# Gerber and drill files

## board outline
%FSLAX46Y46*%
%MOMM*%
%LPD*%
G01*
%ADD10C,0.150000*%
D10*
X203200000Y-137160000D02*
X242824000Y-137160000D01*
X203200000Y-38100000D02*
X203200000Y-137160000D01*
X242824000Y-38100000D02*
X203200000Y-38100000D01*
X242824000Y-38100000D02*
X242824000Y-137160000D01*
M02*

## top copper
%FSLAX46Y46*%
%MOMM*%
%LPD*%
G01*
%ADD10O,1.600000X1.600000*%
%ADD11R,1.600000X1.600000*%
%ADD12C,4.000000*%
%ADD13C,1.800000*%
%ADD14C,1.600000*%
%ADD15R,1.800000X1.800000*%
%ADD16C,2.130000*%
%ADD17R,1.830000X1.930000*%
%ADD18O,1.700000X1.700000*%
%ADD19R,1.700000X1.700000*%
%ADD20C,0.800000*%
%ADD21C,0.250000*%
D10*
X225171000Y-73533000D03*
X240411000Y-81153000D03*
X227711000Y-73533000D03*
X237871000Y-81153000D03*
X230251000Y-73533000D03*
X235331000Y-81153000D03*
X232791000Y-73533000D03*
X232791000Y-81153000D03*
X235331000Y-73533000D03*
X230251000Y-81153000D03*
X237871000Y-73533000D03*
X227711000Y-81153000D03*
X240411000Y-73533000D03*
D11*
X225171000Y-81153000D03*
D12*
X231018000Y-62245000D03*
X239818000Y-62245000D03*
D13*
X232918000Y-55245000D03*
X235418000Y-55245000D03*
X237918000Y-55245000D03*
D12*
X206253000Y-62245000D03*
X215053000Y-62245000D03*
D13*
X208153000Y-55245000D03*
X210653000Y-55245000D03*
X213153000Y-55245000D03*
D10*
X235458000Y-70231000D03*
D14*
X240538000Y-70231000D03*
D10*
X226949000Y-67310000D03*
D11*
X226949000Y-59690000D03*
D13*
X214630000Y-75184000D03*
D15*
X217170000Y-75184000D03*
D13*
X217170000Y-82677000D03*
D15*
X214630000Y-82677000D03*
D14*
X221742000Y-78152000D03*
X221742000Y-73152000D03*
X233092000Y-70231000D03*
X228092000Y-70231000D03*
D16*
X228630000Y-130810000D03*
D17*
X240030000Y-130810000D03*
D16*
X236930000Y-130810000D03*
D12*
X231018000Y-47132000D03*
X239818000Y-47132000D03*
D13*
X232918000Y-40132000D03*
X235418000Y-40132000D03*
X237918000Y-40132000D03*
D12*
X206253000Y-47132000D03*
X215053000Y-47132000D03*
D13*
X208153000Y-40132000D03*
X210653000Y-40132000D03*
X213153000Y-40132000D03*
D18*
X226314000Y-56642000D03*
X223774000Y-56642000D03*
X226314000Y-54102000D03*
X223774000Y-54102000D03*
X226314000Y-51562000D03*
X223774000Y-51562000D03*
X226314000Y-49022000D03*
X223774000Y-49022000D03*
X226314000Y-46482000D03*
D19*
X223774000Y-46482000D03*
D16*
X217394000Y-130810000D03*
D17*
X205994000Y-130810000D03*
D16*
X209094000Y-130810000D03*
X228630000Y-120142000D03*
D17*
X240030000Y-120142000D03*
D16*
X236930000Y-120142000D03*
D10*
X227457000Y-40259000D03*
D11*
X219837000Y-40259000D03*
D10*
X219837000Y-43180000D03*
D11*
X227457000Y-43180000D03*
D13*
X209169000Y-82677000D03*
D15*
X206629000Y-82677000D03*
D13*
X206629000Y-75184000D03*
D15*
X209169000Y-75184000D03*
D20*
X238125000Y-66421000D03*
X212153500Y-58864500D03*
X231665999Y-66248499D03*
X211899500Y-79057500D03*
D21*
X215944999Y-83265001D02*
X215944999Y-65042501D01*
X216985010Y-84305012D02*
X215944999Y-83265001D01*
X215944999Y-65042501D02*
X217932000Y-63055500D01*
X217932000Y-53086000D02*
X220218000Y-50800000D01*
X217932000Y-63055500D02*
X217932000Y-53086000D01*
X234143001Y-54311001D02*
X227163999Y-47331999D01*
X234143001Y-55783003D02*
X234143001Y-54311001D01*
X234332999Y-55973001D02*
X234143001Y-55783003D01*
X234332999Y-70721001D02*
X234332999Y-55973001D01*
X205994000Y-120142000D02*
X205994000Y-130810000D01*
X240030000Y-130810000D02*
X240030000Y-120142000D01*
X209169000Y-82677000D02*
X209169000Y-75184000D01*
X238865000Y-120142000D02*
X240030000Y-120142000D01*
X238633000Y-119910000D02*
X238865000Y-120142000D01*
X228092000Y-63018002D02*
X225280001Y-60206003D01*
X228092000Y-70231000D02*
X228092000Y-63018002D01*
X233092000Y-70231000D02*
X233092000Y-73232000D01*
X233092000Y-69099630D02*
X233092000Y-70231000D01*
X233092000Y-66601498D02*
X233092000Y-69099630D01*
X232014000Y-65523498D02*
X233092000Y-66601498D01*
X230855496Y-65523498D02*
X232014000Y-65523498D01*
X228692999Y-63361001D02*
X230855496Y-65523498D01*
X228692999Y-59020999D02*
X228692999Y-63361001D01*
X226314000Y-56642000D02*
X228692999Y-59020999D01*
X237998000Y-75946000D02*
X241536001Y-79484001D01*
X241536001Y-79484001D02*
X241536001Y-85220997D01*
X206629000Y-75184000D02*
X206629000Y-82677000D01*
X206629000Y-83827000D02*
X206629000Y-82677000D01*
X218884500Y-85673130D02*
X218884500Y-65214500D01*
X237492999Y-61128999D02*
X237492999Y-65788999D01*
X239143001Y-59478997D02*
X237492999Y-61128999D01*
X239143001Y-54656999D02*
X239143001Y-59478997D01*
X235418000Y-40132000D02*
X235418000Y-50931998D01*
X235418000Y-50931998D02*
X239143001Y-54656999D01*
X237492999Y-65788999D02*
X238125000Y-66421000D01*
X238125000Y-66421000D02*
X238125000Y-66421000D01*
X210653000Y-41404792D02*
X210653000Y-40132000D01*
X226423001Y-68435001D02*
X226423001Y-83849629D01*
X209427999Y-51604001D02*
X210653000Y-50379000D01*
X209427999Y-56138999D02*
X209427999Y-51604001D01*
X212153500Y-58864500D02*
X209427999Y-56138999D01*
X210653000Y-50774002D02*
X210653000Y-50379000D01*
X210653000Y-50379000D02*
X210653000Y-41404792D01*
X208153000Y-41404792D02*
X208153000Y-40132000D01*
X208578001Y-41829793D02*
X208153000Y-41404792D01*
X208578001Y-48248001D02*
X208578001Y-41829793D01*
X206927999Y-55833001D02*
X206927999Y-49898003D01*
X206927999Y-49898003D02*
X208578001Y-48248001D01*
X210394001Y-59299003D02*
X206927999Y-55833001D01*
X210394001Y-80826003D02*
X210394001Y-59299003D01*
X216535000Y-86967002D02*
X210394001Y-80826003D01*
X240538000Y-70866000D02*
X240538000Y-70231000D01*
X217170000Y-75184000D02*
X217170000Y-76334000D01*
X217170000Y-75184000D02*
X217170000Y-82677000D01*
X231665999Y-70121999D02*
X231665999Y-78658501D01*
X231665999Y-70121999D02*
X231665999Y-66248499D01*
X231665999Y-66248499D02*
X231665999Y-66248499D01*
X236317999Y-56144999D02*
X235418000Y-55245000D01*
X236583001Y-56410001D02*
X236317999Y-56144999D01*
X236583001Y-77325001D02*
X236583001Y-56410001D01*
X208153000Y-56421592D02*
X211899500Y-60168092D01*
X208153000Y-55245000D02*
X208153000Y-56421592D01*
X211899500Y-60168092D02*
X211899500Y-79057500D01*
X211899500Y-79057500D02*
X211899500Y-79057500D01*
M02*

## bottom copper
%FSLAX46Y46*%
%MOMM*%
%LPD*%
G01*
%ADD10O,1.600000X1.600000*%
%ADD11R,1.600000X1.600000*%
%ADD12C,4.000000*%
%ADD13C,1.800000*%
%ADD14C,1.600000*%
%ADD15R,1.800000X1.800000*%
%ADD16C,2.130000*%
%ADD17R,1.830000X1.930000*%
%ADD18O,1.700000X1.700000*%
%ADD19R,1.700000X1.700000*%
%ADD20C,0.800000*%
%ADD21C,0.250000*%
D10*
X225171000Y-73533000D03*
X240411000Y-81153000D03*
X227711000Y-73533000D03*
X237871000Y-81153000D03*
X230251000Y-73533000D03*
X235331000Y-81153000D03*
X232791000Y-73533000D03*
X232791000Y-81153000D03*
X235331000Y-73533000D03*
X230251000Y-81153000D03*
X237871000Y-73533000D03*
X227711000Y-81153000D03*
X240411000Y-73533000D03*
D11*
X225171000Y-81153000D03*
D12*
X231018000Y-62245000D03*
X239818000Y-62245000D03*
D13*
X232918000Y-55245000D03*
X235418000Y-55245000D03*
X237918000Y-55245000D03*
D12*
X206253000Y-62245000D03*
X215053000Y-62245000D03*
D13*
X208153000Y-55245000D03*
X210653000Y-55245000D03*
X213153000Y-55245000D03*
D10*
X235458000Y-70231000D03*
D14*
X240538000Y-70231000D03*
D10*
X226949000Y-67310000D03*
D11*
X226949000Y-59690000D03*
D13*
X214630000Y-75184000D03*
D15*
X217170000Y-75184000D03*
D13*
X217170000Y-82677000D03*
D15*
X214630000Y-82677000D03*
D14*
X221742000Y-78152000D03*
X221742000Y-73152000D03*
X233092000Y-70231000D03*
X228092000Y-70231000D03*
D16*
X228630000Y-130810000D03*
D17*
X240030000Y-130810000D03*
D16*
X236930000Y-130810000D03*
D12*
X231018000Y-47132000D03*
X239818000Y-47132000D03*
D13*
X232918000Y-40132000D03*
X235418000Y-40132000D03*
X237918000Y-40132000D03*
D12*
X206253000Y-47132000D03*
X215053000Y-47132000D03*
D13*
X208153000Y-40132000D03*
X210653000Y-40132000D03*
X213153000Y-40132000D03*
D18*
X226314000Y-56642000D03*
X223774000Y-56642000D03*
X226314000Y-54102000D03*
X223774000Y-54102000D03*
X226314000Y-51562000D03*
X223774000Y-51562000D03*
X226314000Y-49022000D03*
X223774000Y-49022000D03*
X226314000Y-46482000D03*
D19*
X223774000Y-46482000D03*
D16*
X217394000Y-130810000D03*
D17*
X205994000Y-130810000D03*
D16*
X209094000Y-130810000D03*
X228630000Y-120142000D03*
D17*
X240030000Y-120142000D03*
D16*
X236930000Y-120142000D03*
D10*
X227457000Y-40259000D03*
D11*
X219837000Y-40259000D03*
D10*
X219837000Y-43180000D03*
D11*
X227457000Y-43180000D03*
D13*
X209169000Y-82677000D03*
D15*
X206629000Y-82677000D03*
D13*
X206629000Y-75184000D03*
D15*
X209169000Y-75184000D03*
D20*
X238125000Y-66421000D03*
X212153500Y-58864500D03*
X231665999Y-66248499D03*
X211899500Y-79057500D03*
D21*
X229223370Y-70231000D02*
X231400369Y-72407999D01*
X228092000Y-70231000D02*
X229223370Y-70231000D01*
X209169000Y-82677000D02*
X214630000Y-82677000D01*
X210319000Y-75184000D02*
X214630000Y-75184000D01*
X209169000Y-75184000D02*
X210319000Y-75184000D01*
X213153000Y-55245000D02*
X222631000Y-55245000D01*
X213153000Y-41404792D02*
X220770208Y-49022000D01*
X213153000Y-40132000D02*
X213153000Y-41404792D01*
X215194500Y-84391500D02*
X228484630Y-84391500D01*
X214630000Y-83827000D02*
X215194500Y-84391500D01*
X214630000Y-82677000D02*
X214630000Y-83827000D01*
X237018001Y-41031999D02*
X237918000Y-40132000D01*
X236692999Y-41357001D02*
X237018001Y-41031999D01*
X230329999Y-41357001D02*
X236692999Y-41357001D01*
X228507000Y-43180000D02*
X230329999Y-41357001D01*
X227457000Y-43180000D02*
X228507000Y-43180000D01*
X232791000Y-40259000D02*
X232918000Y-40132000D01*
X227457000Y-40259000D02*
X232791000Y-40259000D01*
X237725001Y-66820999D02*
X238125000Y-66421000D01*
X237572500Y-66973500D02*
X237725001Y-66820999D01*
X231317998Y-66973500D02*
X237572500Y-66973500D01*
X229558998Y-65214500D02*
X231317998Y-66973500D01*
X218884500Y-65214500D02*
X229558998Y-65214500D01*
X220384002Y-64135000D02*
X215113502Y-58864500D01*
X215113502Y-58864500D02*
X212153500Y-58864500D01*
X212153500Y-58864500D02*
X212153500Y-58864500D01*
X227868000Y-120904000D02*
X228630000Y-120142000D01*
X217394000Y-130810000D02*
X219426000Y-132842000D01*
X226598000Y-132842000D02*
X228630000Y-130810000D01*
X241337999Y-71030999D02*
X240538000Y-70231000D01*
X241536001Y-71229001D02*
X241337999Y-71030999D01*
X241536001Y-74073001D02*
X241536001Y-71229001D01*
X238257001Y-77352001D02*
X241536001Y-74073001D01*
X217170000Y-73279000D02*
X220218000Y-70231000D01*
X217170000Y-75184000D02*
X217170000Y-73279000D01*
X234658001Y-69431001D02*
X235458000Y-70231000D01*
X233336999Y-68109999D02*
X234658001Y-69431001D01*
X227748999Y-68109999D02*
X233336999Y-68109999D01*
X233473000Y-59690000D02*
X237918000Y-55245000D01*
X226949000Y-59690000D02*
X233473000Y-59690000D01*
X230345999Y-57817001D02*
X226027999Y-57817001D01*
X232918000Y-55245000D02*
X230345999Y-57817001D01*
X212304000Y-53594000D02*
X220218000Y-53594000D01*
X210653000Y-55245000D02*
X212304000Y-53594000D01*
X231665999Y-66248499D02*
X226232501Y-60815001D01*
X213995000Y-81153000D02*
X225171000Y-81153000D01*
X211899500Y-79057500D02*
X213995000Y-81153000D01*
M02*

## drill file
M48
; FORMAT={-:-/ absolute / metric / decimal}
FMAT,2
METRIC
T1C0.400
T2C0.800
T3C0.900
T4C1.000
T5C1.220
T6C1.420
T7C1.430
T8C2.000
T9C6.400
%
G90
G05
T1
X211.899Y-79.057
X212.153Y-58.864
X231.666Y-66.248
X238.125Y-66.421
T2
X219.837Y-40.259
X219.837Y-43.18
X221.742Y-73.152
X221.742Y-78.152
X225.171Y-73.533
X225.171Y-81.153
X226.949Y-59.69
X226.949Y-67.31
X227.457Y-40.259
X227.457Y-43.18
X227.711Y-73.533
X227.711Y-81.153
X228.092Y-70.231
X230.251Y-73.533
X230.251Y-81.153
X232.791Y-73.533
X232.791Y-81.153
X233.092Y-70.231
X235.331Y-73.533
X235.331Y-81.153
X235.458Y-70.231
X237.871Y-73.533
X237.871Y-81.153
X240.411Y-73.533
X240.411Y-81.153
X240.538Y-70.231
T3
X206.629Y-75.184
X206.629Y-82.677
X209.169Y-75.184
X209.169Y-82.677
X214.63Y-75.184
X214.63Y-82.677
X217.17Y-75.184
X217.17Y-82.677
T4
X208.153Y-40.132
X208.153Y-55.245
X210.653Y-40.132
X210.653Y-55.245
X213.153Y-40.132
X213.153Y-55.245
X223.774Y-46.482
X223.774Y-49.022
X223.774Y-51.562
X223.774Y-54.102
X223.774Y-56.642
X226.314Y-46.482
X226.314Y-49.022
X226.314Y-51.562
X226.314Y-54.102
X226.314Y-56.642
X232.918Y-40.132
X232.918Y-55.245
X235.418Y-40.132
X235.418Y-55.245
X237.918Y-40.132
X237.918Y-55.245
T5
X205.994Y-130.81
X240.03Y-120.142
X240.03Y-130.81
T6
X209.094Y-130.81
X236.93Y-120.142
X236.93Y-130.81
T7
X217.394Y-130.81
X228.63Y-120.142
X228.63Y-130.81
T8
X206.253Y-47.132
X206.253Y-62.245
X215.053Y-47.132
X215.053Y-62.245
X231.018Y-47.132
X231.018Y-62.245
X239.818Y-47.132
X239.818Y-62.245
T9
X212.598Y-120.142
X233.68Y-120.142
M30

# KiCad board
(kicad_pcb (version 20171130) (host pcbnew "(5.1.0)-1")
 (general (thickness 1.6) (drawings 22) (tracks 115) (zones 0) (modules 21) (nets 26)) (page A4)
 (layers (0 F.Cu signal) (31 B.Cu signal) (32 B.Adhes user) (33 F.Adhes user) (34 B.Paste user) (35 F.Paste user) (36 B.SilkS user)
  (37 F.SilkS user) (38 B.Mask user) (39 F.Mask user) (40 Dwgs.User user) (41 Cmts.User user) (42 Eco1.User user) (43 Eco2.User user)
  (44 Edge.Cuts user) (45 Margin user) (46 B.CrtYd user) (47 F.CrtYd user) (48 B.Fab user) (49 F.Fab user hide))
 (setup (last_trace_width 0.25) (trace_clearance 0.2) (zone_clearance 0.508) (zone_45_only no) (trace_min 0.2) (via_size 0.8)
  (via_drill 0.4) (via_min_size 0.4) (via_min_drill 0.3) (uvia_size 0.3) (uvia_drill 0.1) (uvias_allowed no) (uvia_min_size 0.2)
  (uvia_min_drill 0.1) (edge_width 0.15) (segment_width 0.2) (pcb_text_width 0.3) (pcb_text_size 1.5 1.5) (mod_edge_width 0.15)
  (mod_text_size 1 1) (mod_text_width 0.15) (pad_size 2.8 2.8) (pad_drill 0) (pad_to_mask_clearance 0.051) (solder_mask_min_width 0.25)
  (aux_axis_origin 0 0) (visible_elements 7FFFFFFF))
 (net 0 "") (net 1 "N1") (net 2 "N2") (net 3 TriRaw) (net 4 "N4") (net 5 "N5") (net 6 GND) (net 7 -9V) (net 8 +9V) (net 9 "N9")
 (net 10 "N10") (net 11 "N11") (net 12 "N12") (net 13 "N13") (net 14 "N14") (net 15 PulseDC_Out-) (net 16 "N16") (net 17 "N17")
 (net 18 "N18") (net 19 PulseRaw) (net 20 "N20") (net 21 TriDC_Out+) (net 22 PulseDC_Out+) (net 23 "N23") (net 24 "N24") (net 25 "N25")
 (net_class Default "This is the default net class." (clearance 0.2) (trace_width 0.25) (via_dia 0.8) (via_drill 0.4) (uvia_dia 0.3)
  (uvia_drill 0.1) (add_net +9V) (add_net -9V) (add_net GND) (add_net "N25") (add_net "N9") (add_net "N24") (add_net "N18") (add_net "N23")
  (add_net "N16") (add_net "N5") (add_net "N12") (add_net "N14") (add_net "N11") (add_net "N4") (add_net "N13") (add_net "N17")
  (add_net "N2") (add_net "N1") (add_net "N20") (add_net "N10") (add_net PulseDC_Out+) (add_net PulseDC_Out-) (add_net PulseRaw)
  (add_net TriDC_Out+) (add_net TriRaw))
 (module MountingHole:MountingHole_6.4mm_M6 (layer F.Cu) (at 233.68 120.142)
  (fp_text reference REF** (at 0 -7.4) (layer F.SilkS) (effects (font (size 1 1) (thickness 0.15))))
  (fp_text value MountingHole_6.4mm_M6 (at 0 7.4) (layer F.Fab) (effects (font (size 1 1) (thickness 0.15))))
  (pad 1 np_thru_hole circle (at 0 0) (size 6.4 6.4) (drill 6.4) (layers *.Cu *.Mask)))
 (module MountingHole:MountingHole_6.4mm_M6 (layer F.Cu) (at 212.598 120.142)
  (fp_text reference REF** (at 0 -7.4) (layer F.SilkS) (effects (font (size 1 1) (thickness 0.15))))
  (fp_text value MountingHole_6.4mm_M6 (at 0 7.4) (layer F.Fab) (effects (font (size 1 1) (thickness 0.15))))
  (pad 1 np_thru_hole circle (at 0 0) (size 6.4 6.4) (drill 6.4) (layers *.Cu *.Mask)))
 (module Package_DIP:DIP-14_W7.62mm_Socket (layer F.Cu) (at 225.171 81.153 90)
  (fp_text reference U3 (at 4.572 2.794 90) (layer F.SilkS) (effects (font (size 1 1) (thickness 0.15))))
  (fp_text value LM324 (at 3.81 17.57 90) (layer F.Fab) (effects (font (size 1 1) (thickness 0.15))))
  (pad 14 thru_hole oval (at 7.62 0 90) (size 1.6 1.6) (drill 0.8) (layers *.Cu *.Mask) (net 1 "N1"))
  (pad 7 thru_hole oval (at 0 15.24 90) (size 1.6 1.6) (drill 0.8) (layers *.Cu *.Mask) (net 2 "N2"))
  (pad 13 thru_hole oval (at 7.62 2.54 90) (size 1.6 1.6) (drill 0.8) (layers *.Cu *.Mask) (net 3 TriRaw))
  (pad 6 thru_hole oval (at 0 12.7 90) (size 1.6 1.6) (drill 0.8) (layers *.Cu *.Mask) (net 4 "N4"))
  (pad 12 thru_hole oval (at 7.62 5.08 90) (size 1.6 1.6) (drill 0.8) (layers *.Cu *.Mask) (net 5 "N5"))
  (pad 5 thru_hole oval (at 0 10.16 90) (size 1.6 1.6) (drill 0.8) (layers *.Cu *.Mask) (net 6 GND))
  (pad 11 thru_hole oval (at 7.62 7.62 90) (size 1.6 1.6) (drill 0.8) (layers *.Cu *.Mask) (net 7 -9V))
  (pad 4 thru_hole oval (at 0 7.62 90) (size 1.6 1.6) (drill 0.8) (layers *.Cu *.Mask) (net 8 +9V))
  (pad 10 thru_hole oval (at 7.62 10.16 90) (size 1.6 1.6) (drill 0.8) (layers *.Cu *.Mask) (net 6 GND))
  (pad 3 thru_hole oval (at 0 5.08 90) (size 1.6 1.6) (drill 0.8) (layers *.Cu *.Mask) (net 5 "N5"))
  (pad 9 thru_hole oval (at 7.62 12.7 90) (size 1.6 1.6) (drill 0.8) (layers *.Cu *.Mask) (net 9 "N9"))
  (pad 2 thru_hole oval (at 0 2.54 90) (size 1.6 1.6) (drill 0.8) (layers *.Cu *.Mask) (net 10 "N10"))
  (pad 8 thru_hole oval (at 7.62 15.24 90) (size 1.6 1.6) (drill 0.8) (layers *.Cu *.Mask) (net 3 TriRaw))
  (pad 1 thru_hole rect (at 0 0 90) (size 1.6 1.6) (drill 0.8) (layers *.Cu *.Mask) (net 10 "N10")))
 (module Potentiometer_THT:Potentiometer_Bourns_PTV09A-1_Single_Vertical (layer F.Cu) (at 232.918 55.245 270)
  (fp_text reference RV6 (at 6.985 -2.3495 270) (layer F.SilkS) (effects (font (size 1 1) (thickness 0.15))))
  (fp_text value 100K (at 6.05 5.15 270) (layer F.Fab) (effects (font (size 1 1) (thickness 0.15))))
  (pad "" np_thru_hole circle (at 7 1.9 270) (size 4 4) (drill 2) (layers *.Cu *.Mask))
  (pad "" np_thru_hole circle (at 7 -6.9 270) (size 4 4) (drill 2) (layers *.Cu *.Mask))
  (pad 1 thru_hole circle (at 0 0 270) (size 1.8 1.8) (drill 1) (layers *.Cu *.Mask) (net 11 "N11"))
  (pad 2 thru_hole circle (at 0 -2.5 270) (size 1.8 1.8) (drill 1) (layers *.Cu *.Mask) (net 2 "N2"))
  (pad 3 thru_hole circle (at 0 -5 270) (size 1.8 1.8) (drill 1) (layers *.Cu *.Mask) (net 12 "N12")))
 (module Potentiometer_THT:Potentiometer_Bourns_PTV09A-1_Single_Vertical (layer F.Cu) (at 208.153 55.245 270)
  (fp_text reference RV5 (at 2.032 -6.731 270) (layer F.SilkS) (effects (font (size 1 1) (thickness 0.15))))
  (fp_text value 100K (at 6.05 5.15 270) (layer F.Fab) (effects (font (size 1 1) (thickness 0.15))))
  (pad "" np_thru_hole circle (at 7 1.9 270) (size 4 4) (drill 2) (layers *.Cu *.Mask))
  (pad "" np_thru_hole circle (at 7 -6.9 270) (size 4 4) (drill 2) (layers *.Cu *.Mask))
  (pad 1 thru_hole circle (at 0 0 270) (size 1.8 1.8) (drill 1) (layers *.Cu *.Mask) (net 10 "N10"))
  (pad 2 thru_hole circle (at 0 -2.5 270) (size 1.8 1.8) (drill 1) (layers *.Cu *.Mask) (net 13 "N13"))
  (pad 3 thru_hole circle (at 0 -5 270) (size 1.8 1.8) (drill 1) (layers *.Cu *.Mask) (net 6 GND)))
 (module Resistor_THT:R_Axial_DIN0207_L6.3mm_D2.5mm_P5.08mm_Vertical (layer F.Cu) (at 240.538 70.231 180)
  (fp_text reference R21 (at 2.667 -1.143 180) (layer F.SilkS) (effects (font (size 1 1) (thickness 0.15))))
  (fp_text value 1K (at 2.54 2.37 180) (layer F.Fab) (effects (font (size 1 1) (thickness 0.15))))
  (pad 2 thru_hole oval (at 5.08 0 180) (size 1.6 1.6) (drill 0.8) (layers *.Cu *.Mask) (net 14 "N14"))
  (pad 1 thru_hole circle (at 0 0 180) (size 1.6 1.6) (drill 0.8) (layers *.Cu *.Mask) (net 9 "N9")))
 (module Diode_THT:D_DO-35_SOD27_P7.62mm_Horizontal (layer F.Cu) (at 226.949 59.69 270)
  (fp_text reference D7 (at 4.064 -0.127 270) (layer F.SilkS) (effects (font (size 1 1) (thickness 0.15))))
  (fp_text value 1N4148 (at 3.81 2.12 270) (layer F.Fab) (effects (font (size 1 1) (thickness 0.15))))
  (pad 2 thru_hole oval (at 7.62 0 270) (size 1.6 1.6) (drill 0.8) (layers *.Cu *.Mask) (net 14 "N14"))
  (pad 1 thru_hole rect (at 0 0 270) (size 1.6 1.6) (drill 0.8) (layers *.Cu *.Mask) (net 12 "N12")))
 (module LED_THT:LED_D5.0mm (layer F.Cu) (at 217.17 75.184 180)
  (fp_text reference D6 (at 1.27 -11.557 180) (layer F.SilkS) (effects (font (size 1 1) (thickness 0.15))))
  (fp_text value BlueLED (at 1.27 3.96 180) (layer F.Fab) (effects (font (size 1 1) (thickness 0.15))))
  (pad 2 thru_hole circle (at 2.54 0 180) (size 1.8 1.8) (drill 0.9) (layers *.Cu *.Mask) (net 6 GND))
  (pad 1 thru_hole rect (at 0 0 180) (size 1.8 1.8) (drill 0.9) (layers *.Cu *.Mask) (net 5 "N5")))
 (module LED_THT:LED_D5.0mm (layer F.Cu) (at 214.63 82.677)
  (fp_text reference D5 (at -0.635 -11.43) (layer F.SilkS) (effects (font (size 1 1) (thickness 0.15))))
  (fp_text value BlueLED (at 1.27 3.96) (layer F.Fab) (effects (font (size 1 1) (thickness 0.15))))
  (pad 2 thru_hole circle (at 2.54 0) (size 1.8 1.8) (drill 0.9) (layers *.Cu *.Mask) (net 5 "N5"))
  (pad 1 thru_hole rect (at 0 0) (size 1.8 1.8) (drill 0.9) (layers *.Cu *.Mask) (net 6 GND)))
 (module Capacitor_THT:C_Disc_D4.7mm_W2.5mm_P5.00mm (layer F.Cu) (at 221.742 73.152 270)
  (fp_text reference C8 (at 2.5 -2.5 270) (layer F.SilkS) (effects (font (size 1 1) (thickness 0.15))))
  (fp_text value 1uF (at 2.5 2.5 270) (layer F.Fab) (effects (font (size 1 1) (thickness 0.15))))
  (pad 2 thru_hole circle (at 5 0 270) (size 1.6 1.6) (drill 0.8) (layers *.Cu *.Mask) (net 9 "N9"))
  (pad 1 thru_hole circle (at 0 0 270) (size 1.6 1.6) (drill 0.8) (layers *.Cu *.Mask) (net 3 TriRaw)))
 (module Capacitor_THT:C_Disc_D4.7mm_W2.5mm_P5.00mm (layer F.Cu) (at 228.092 70.231)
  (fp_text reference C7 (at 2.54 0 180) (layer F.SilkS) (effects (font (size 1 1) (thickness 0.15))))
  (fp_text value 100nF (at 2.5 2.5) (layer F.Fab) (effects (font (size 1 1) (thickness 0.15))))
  (pad 2 thru_hole circle (at 5 0) (size 1.6 1.6) (drill 0.8) (layers *.Cu *.Mask) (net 7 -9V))
  (pad 1 thru_hole circle (at 0 0) (size 1.6 1.6) (drill 0.8) (layers *.Cu *.Mask) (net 6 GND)))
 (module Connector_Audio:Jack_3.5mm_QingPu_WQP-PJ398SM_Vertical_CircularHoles (layer F.Cu) (at 240.03 130.81 270)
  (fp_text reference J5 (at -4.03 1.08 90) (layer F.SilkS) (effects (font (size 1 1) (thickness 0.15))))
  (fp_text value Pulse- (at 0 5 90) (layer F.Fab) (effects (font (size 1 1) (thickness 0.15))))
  (pad T thru_hole circle (at 0 11.4 90) (size 2.13 2.13) (drill 1.43) (layers *.Cu *.Mask) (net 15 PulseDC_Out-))
  (pad S thru_hole rect (at 0 0 90) (size 1.93 1.83) (drill 1.22) (layers *.Cu *.Mask) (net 6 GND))
  (pad TN thru_hole circle (at 0 3.1 90) (size 2.13 2.13) (drill 1.42) (layers *.Cu *.Mask)))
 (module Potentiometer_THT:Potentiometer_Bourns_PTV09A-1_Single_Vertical (layer F.Cu) (at 232.918 40.132 270)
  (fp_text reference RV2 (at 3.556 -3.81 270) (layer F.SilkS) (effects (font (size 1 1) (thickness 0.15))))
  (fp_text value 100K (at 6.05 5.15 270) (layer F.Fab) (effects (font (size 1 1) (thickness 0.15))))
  (pad "" np_thru_hole circle (at 7 1.9 270) (size 4 4) (drill 2) (layers *.Cu *.Mask))
  (pad "" np_thru_hole circle (at 7 -6.9 270) (size 4 4) (drill 2) (layers *.Cu *.Mask))
  (pad 1 thru_hole circle (at 0 0 270) (size 1.8 1.8) (drill 1) (layers *.Cu *.Mask) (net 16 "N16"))
  (pad 2 thru_hole circle (at 0 -2.5 270) (size 1.8 1.8) (drill 1) (layers *.Cu *.Mask) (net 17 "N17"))
  (pad 3 thru_hole circle (at 0 -5 270) (size 1.8 1.8) (drill 1) (layers *.Cu *.Mask) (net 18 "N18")))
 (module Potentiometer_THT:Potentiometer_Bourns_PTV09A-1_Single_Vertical (layer F.Cu) (at 208.153 40.132 270)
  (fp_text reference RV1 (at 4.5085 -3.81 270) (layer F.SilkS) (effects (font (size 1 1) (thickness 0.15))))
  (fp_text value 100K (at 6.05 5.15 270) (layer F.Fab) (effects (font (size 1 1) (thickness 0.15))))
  (pad "" np_thru_hole circle (at 7 1.9 270) (size 4 4) (drill 2) (layers *.Cu *.Mask))
  (pad "" np_thru_hole circle (at 7 -6.9 270) (size 4 4) (drill 2) (layers *.Cu *.Mask))
  (pad 1 thru_hole circle (at 0 0 270) (size 1.8 1.8) (drill 1) (layers *.Cu *.Mask) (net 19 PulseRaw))
  (pad 2 thru_hole circle (at 0 -2.5 270) (size 1.8 1.8) (drill 1) (layers *.Cu *.Mask) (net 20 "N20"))
  (pad 3 thru_hole circle (at 0 -5 270) (size 1.8 1.8) (drill 1) (layers *.Cu *.Mask) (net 6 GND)))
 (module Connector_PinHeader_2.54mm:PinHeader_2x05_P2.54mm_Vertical (layer F.Cu) (at 223.774 46.482)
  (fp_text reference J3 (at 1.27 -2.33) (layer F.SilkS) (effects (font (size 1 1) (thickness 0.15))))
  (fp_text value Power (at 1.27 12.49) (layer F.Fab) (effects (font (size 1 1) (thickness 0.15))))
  (pad 10 thru_hole oval (at 2.54 10.16) (size 1.7 1.7) (drill 1) (layers *.Cu *.Mask) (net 7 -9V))
  (pad 9 thru_hole oval (at 0 10.16) (size 1.7 1.7) (drill 1) (layers *.Cu *.Mask) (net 7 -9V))
  (pad 8 thru_hole oval (at 2.54 7.62) (size 1.7 1.7) (drill 1) (layers *.Cu *.Mask) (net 6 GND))
  (pad 7 thru_hole oval (at 0 7.62) (size 1.7 1.7) (drill 1) (layers *.Cu *.Mask) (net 6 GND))
  (pad 6 thru_hole oval (at 2.54 5.08) (size 1.7 1.7) (drill 1) (layers *.Cu *.Mask) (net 6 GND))
  (pad 5 thru_hole oval (at 0 5.08) (size 1.7 1.7) (drill 1) (layers *.Cu *.Mask) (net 6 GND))
  (pad 4 thru_hole oval (at 2.54 2.54) (size 1.7 1.7) (drill 1) (layers *.Cu *.Mask) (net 6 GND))
  (pad 3 thru_hole oval (at 0 2.54) (size 1.7 1.7) (drill 1) (layers *.Cu *.Mask) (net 6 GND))
  (pad 2 thru_hole oval (at 2.54 0) (size 1.7 1.7) (drill 1) (layers *.Cu *.Mask) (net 8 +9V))
  (pad 1 thru_hole rect (at 0 0) (size 1.7 1.7) (drill 1) (layers *.Cu *.Mask) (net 8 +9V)))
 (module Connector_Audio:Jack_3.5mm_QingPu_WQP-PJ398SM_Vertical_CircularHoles (layer F.Cu) (at 205.994 130.81 90)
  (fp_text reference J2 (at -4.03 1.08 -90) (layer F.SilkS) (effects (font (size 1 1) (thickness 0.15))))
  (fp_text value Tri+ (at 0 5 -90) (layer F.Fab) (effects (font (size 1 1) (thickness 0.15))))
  (pad T thru_hole circle (at 0 11.4 270) (size 2.13 2.13) (drill 1.43) (layers *.Cu *.Mask) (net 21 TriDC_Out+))
  (pad S thru_hole rect (at 0 0 270) (size 1.93 1.83) (drill 1.22) (layers *.Cu *.Mask) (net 6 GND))
  (pad TN thru_hole circle (at 0 3.1 270) (size 2.13 2.13) (drill 1.42) (layers *.Cu *.Mask)))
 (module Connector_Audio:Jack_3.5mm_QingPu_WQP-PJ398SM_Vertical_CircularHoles (layer F.Cu) (at 240.03 120.142 270)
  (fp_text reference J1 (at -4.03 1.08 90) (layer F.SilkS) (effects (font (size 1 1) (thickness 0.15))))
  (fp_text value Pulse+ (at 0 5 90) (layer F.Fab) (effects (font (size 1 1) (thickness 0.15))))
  (pad T thru_hole circle (at 0 11.4 90) (size 2.13 2.13) (drill 1.43) (layers *.Cu *.Mask) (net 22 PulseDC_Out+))
  (pad S thru_hole rect (at 0 0 90) (size 1.93 1.83) (drill 1.22) (layers *.Cu *.Mask) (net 6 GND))
  (pad TN thru_hole circle (at 0 3.1 90) (size 2.13 2.13) (drill 1.42) (layers *.Cu *.Mask)))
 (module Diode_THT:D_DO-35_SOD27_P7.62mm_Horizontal (layer F.Cu) (at 219.837 40.259)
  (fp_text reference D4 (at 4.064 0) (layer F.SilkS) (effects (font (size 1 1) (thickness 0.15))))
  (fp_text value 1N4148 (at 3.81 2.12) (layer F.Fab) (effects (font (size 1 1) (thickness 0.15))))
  (pad 2 thru_hole oval (at 7.62 0) (size 1.6 1.6) (drill 0.8) (layers *.Cu *.Mask) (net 16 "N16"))
  (pad 1 thru_hole rect (at 0 0) (size 1.6 1.6) (drill 0.8) (layers *.Cu *.Mask) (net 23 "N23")))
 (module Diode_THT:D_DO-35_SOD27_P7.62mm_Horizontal (layer F.Cu) (at 227.457 43.18 180)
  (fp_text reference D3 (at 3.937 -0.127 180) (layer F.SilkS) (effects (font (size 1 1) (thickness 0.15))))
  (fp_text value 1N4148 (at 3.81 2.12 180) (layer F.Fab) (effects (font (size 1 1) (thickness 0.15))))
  (pad 2 thru_hole oval (at 7.62 0 180) (size 1.6 1.6) (drill 0.8) (layers *.Cu *.Mask) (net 23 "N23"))
  (pad 1 thru_hole rect (at 0 0 180) (size 1.6 1.6) (drill 0.8) (layers *.Cu *.Mask) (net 18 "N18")))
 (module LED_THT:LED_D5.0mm (layer F.Cu) (at 206.629 82.677)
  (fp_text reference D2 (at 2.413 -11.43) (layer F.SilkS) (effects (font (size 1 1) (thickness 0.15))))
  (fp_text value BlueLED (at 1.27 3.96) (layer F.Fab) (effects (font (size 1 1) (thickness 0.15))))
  (pad 2 thru_hole circle (at 2.54 0) (size 1.8 1.8) (drill 0.9) (layers *.Cu *.Mask) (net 6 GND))
  (pad 1 thru_hole rect (at 0 0) (size 1.8 1.8) (drill 0.9) (layers *.Cu *.Mask) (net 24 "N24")))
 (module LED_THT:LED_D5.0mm (layer F.Cu) (at 209.169 75.184 180)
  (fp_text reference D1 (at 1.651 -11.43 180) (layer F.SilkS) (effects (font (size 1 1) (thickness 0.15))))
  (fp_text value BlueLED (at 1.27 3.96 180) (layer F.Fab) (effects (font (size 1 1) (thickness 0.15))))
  (pad 2 thru_hole circle (at 2.54 0 180) (size 1.8 1.8) (drill 0.9) (layers *.Cu *.Mask) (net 24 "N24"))
  (pad 1 thru_hole rect (at 0 0 180) (size 1.8 1.8) (drill 0.9) (layers *.Cu *.Mask) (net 6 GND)))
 (gr_line (start 203.2 137.16) (end 242.824 137.16) (layer Edge.Cuts) (width 0.15))
 (gr_line (start 203.2 38.1) (end 203.2 137.16) (layer Edge.Cuts) (width 0.15))
 (gr_line (start 242.824 38.1) (end 203.2 38.1) (layer Edge.Cuts) (width 0.15))
 (gr_line (start 242.824 38.1) (end 242.824 137.16) (layer Edge.Cuts) (width 0.15))
 (segment (start 215.944999 83.265001) (end 215.944999 65.042501) (width 0.25) (layer F.Cu) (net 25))
 (segment (start 216.98501 84.305012) (end 215.944999 83.265001) (width 0.25) (layer F.Cu) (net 25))
 (segment (start 215.944999 65.042501) (end 217.932 63.0555) (width 0.25) (layer F.Cu) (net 25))
 (segment (start 217.932 53.086) (end 220.218 50.8) (width 0.25) (layer F.Cu) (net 25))
 (segment (start 217.932 63.0555) (end 217.932 53.086) (width 0.25) (layer F.Cu) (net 25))
 (segment (start 234.143001 54.311001) (end 227.163999 47.331999) (width 0.25) (layer F.Cu) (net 8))
 (segment (start 234.143001 55.783003) (end 234.143001 54.311001) (width 0.25) (layer F.Cu) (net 8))
 (segment (start 234.332999 55.973001) (end 234.143001 55.783003) (width 0.25) (layer F.Cu) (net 8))
 (segment (start 234.332999 70.721001) (end 234.332999 55.973001) (width 0.25) (layer F.Cu) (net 8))
 (segment (start 205.994 120.142) (end 205.994 130.81) (width 0.25) (layer F.Cu) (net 6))
 (segment (start 240.03 130.81) (end 240.03 120.142) (width 0.25) (layer F.Cu) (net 6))
 (segment (start 229.22337 70.231) (end 231.400369 72.407999) (width 0.25) (layer B.Cu) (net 6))
 (segment (start 228.092 70.231) (end 229.22337 70.231) (width 0.25) (layer B.Cu) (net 6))
 (segment (start 209.169 82.677) (end 209.169 75.184) (width 0.25) (layer F.Cu) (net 6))
 (segment (start 238.865 120.142) (end 240.03 120.142) (width 0.25) (layer F.Cu) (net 6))
 (segment (start 238.633 119.91) (end 238.865 120.142) (width 0.25) (layer F.Cu) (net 6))
 (segment (start 209.169 82.677) (end 214.63 82.677) (width 0.25) (layer B.Cu) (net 6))
 (segment (start 210.319 75.184) (end 214.63 75.184) (width 0.25) (layer B.Cu) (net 6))
 (segment (start 209.169 75.184) (end 210.319 75.184) (width 0.25) (layer B.Cu) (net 6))
 (segment (start 228.092 63.018002) (end 225.280001 60.206003) (width 0.25) (layer F.Cu) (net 6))
 (segment (start 228.092 70.231) (end 228.092 63.018002) (width 0.25) (layer F.Cu) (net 6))
 (segment (start 213.153 55.245) (end 222.631 55.245) (width 0.25) (layer B.Cu) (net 6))
 (segment (start 213.153 41.404792) (end 220.770208 49.022) (width 0.25) (layer B.Cu) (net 6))
 (segment (start 213.153 40.132) (end 213.153 41.404792) (width 0.25) (layer B.Cu) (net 6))
 (segment (start 215.1945 84.3915) (end 228.48463 84.3915) (width 0.25) (layer B.Cu) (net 6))
 (segment (start 214.63 83.827) (end 215.1945 84.3915) (width 0.25) (layer B.Cu) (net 6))
 (segment (start 214.63 82.677) (end 214.63 83.827) (width 0.25) (layer B.Cu) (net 6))
 (segment (start 233.092 70.231) (end 233.092 73.232) (width 0.25) (layer F.Cu) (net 7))
 (segment (start 233.092 69.09963) (end 233.092 70.231) (width 0.25) (layer F.Cu) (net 7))
 (segment (start 233.092 66.601498) (end 233.092 69.09963) (width 0.25) (layer F.Cu) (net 7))
 (segment (start 232.014 65.523498) (end 233.092 66.601498) (width 0.25) (layer F.Cu) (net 7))
 (segment (start 230.855496 65.523498) (end 232.014 65.523498) (width 0.25) (layer F.Cu) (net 7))
 (segment (start 228.692999 63.361001) (end 230.855496 65.523498) (width 0.25) (layer F.Cu) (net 7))
 (segment (start 228.692999 59.020999) (end 228.692999 63.361001) (width 0.25) (layer F.Cu) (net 7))
 (segment (start 226.314 56.642) (end 228.692999 59.020999) (width 0.25) (layer F.Cu) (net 7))
 (segment (start 237.998 75.946) (end 241.536001 79.484001) (width 0.25) (layer F.Cu) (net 7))
 (segment (start 241.536001 79.484001) (end 241.536001 85.220997) (width 0.25) (layer F.Cu) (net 7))
 (segment (start 206.629 75.184) (end 206.629 82.677) (width 0.25) (layer F.Cu) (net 24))
 (segment (start 206.629 83.827) (end 206.629 82.677) (width 0.25) (layer F.Cu) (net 24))
 (segment (start 237.018001 41.031999) (end 237.918 40.132) (width 0.25) (layer B.Cu) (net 18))
 (segment (start 236.692999 41.357001) (end 237.018001 41.031999) (width 0.25) (layer B.Cu) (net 18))
 (segment (start 230.329999 41.357001) (end 236.692999 41.357001) (width 0.25) (layer B.Cu) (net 18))
 (segment (start 228.507 43.18) (end 230.329999 41.357001) (width 0.25) (layer B.Cu) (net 18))
 (segment (start 227.457 43.18) (end 228.507 43.18) (width 0.25) (layer B.Cu) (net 18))
 (segment (start 232.791 40.259) (end 232.918 40.132) (width 0.25) (layer B.Cu) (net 16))
 (segment (start 227.457 40.259) (end 232.791 40.259) (width 0.25) (layer B.Cu) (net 16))
 (segment (start 218.8845 85.67313) (end 218.8845 65.2145) (width 0.25) (layer F.Cu) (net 17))
 (segment (start 237.492999 61.128999) (end 237.492999 65.788999) (width 0.25) (layer F.Cu) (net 17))
 (segment (start 239.143001 59.478997) (end 237.492999 61.128999) (width 0.25) (layer F.Cu) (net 17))
 (segment (start 239.143001 54.656999) (end 239.143001 59.478997) (width 0.25) (layer F.Cu) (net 17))
 (segment (start 235.418 40.132) (end 235.418 50.931998) (width 0.25) (layer F.Cu) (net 17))
 (segment (start 235.418 50.931998) (end 239.143001 54.656999) (width 0.25) (layer F.Cu) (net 17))
 (segment (start 237.492999 65.788999) (end 238.125 66.421) (width 0.25) (layer F.Cu) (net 17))
 (segment (start 238.125 66.421) (end 238.125 66.421) (width 0.25) (layer F.Cu) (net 17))
 (via (at 238.125 66.421) (size 0.8) (drill 0.4) (layers F.Cu B.Cu) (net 17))
 (segment (start 237.725001 66.820999) (end 238.125 66.421) (width 0.25) (layer B.Cu) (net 17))
 (segment (start 237.5725 66.9735) (end 237.725001 66.820999) (width 0.25) (layer B.Cu) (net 17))
 (segment (start 231.317998 66.9735) (end 237.5725 66.9735) (width 0.25) (layer B.Cu) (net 17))
 (segment (start 229.558998 65.2145) (end 231.317998 66.9735) (width 0.25) (layer B.Cu) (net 17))
 (segment (start 218.8845 65.2145) (end 229.558998 65.2145) (width 0.25) (layer B.Cu) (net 17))
 (segment (start 210.653 41.404792) (end 210.653 40.132) (width 0.25) (layer F.Cu) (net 20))
 (segment (start 226.423001 68.435001) (end 226.423001 83.849629) (width 0.25) (layer F.Cu) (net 20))
 (segment (start 220.384002 64.135) (end 215.113502 58.8645) (width 0.25) (layer B.Cu) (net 20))
 (segment (start 215.113502 58.8645) (end 212.1535 58.8645) (width 0.25) (layer B.Cu) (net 20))
 (segment (start 212.1535 58.8645) (end 212.1535 58.8645) (width 0.25) (layer B.Cu) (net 20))
 (via (at 212.1535 58.8645) (size 0.8) (drill 0.4) (layers F.Cu B.Cu) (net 20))
 (segment (start 209.427999 51.604001) (end 210.653 50.379) (width 0.25) (layer F.Cu) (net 20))
 (segment (start 209.427999 56.138999) (end 209.427999 51.604001) (width 0.25) (layer F.Cu) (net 20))
 (segment (start 212.1535 58.8645) (end 209.427999 56.138999) (width 0.25) (layer F.Cu) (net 20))
 (segment (start 210.653 50.774002) (end 210.653 50.379) (width 0.25) (layer F.Cu) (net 20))
 (segment (start 210.653 50.379) (end 210.653 41.404792) (width 0.25) (layer F.Cu) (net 20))
 (segment (start 227.868 120.904) (end 228.63 120.142) (width 0.25) (layer B.Cu) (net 22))
 (segment (start 217.394 130.81) (end 219.426 132.842) (width 0.25) (layer B.Cu) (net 21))
 (segment (start 208.153 41.404792) (end 208.153 40.132) (width 0.25) (layer F.Cu) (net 19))
 (segment (start 208.578001 41.829793) (end 208.153 41.404792) (width 0.25) (layer F.Cu) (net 19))
 (segment (start 208.578001 48.248001) (end 208.578001 41.829793) (width 0.25) (layer F.Cu) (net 19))
 (segment (start 206.927999 55.833001) (end 206.927999 49.898003) (width 0.25) (layer F.Cu) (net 19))
 (segment (start 206.927999 49.898003) (end 208.578001 48.248001) (width 0.25) (layer F.Cu) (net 19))
 (segment (start 210.394001 59.299003) (end 206.927999 55.833001) (width 0.25) (layer F.Cu) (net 19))
 (segment (start 210.394001 80.826003) (end 210.394001 59.299003) (width 0.25) (layer F.Cu) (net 19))
 (segment (start 216.535 86.967002) (end 210.394001 80.826003) (width 0.25) (layer F.Cu) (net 19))
 (segment (start 226.598 132.842) (end 228.63 130.81) (width 0.25) (layer B.Cu) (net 15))
 (segment (start 240.538 70.866) (end 240.538 70.231) (width 0.25) (layer F.Cu) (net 9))
 (segment (start 241.337999 71.030999) (end 240.538 70.231) (width 0.25) (layer B.Cu) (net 9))
 (segment (start 241.536001 71.229001) (end 241.337999 71.030999) (width 0.25) (layer B.Cu) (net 9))
 (segment (start 241.536001 74.073001) (end 241.536001 71.229001) (width 0.25) (layer B.Cu) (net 9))
 (segment (start 238.257001 77.352001) (end 241.536001 74.073001) (width 0.25) (layer B.Cu) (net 9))
 (segment (start 217.17 75.184) (end 217.17 76.334) (width 0.25) (layer F.Cu) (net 5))
 (segment (start 217.17 73.279) (end 220.218 70.231) (width 0.25) (layer B.Cu) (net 5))
 (segment (start 217.17 75.184) (end 217.17 73.279) (width 0.25) (layer B.Cu) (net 5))
 (segment (start 217.17 75.184) (end 217.17 82.677) (width 0.25) (layer F.Cu) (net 5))
 (segment (start 234.658001 69.431001) (end 235.458 70.231) (width 0.25) (layer B.Cu) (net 14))
 (segment (start 233.336999 68.109999) (end 234.658001 69.431001) (width 0.25) (layer B.Cu) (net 14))
 (segment (start 227.748999 68.109999) (end 233.336999 68.109999) (width 0.25) (layer B.Cu) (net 14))
 (segment (start 233.473 59.69) (end 237.918 55.245) (width 0.25) (layer B.Cu) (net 12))
 (segment (start 226.949 59.69) (end 233.473 59.69) (width 0.25) (layer B.Cu) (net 12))
 (segment (start 230.345999 57.817001) (end 226.027999 57.817001) (width 0.25) (layer B.Cu) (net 11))
 (segment (start 232.918 55.245) (end 230.345999 57.817001) (width 0.25) (layer B.Cu) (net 11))
 (segment (start 212.304 53.594) (end 220.218 53.594) (width 0.25) (layer B.Cu) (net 13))
 (segment (start 210.653 55.245) (end 212.304 53.594) (width 0.25) (layer B.Cu) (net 13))
 (segment (start 231.665999 70.121999) (end 231.665999 78.658501) (width 0.25) (layer F.Cu) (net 4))
 (segment (start 231.665999 70.121999) (end 231.665999 66.248499) (width 0.25) (layer F.Cu) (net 4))
 (segment (start 231.665999 66.248499) (end 231.665999 66.248499) (width 0.25) (layer F.Cu) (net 4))
 (via (at 231.665999 66.248499) (size 0.8) (drill 0.4) (layers F.Cu B.Cu) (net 4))
 (segment (start 231.665999 66.248499) (end 226.232501 60.815001) (width 0.25) (layer B.Cu) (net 4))
 (segment (start 236.317999 56.144999) (end 235.418 55.245) (width 0.25) (layer F.Cu) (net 2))
 (segment (start 236.583001 56.410001) (end 236.317999 56.144999) (width 0.25) (layer F.Cu) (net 2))
 (segment (start 236.583001 77.325001) (end 236.583001 56.410001) (width 0.25) (layer F.Cu) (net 2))
 (segment (start 208.153 56.421592) (end 211.8995 60.168092) (width 0.25) (layer F.Cu) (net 10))
 (segment (start 208.153 55.245) (end 208.153 56.421592) (width 0.25) (layer F.Cu) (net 10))
 (segment (start 211.8995 60.168092) (end 211.8995 79.0575) (width 0.25) (layer F.Cu) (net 10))
 (segment (start 211.8995 79.0575) (end 211.8995 79.0575) (width 0.25) (layer F.Cu) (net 10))
 (via (at 211.8995 79.0575) (size 0.8) (drill 0.4) (layers F.Cu B.Cu) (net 10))
 (segment (start 213.995 81.153) (end 225.171 81.153) (width 0.25) (layer B.Cu) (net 10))
 (segment (start 211.8995 79.0575) (end 213.995 81.153) (width 0.25) (layer B.Cu) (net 10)))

